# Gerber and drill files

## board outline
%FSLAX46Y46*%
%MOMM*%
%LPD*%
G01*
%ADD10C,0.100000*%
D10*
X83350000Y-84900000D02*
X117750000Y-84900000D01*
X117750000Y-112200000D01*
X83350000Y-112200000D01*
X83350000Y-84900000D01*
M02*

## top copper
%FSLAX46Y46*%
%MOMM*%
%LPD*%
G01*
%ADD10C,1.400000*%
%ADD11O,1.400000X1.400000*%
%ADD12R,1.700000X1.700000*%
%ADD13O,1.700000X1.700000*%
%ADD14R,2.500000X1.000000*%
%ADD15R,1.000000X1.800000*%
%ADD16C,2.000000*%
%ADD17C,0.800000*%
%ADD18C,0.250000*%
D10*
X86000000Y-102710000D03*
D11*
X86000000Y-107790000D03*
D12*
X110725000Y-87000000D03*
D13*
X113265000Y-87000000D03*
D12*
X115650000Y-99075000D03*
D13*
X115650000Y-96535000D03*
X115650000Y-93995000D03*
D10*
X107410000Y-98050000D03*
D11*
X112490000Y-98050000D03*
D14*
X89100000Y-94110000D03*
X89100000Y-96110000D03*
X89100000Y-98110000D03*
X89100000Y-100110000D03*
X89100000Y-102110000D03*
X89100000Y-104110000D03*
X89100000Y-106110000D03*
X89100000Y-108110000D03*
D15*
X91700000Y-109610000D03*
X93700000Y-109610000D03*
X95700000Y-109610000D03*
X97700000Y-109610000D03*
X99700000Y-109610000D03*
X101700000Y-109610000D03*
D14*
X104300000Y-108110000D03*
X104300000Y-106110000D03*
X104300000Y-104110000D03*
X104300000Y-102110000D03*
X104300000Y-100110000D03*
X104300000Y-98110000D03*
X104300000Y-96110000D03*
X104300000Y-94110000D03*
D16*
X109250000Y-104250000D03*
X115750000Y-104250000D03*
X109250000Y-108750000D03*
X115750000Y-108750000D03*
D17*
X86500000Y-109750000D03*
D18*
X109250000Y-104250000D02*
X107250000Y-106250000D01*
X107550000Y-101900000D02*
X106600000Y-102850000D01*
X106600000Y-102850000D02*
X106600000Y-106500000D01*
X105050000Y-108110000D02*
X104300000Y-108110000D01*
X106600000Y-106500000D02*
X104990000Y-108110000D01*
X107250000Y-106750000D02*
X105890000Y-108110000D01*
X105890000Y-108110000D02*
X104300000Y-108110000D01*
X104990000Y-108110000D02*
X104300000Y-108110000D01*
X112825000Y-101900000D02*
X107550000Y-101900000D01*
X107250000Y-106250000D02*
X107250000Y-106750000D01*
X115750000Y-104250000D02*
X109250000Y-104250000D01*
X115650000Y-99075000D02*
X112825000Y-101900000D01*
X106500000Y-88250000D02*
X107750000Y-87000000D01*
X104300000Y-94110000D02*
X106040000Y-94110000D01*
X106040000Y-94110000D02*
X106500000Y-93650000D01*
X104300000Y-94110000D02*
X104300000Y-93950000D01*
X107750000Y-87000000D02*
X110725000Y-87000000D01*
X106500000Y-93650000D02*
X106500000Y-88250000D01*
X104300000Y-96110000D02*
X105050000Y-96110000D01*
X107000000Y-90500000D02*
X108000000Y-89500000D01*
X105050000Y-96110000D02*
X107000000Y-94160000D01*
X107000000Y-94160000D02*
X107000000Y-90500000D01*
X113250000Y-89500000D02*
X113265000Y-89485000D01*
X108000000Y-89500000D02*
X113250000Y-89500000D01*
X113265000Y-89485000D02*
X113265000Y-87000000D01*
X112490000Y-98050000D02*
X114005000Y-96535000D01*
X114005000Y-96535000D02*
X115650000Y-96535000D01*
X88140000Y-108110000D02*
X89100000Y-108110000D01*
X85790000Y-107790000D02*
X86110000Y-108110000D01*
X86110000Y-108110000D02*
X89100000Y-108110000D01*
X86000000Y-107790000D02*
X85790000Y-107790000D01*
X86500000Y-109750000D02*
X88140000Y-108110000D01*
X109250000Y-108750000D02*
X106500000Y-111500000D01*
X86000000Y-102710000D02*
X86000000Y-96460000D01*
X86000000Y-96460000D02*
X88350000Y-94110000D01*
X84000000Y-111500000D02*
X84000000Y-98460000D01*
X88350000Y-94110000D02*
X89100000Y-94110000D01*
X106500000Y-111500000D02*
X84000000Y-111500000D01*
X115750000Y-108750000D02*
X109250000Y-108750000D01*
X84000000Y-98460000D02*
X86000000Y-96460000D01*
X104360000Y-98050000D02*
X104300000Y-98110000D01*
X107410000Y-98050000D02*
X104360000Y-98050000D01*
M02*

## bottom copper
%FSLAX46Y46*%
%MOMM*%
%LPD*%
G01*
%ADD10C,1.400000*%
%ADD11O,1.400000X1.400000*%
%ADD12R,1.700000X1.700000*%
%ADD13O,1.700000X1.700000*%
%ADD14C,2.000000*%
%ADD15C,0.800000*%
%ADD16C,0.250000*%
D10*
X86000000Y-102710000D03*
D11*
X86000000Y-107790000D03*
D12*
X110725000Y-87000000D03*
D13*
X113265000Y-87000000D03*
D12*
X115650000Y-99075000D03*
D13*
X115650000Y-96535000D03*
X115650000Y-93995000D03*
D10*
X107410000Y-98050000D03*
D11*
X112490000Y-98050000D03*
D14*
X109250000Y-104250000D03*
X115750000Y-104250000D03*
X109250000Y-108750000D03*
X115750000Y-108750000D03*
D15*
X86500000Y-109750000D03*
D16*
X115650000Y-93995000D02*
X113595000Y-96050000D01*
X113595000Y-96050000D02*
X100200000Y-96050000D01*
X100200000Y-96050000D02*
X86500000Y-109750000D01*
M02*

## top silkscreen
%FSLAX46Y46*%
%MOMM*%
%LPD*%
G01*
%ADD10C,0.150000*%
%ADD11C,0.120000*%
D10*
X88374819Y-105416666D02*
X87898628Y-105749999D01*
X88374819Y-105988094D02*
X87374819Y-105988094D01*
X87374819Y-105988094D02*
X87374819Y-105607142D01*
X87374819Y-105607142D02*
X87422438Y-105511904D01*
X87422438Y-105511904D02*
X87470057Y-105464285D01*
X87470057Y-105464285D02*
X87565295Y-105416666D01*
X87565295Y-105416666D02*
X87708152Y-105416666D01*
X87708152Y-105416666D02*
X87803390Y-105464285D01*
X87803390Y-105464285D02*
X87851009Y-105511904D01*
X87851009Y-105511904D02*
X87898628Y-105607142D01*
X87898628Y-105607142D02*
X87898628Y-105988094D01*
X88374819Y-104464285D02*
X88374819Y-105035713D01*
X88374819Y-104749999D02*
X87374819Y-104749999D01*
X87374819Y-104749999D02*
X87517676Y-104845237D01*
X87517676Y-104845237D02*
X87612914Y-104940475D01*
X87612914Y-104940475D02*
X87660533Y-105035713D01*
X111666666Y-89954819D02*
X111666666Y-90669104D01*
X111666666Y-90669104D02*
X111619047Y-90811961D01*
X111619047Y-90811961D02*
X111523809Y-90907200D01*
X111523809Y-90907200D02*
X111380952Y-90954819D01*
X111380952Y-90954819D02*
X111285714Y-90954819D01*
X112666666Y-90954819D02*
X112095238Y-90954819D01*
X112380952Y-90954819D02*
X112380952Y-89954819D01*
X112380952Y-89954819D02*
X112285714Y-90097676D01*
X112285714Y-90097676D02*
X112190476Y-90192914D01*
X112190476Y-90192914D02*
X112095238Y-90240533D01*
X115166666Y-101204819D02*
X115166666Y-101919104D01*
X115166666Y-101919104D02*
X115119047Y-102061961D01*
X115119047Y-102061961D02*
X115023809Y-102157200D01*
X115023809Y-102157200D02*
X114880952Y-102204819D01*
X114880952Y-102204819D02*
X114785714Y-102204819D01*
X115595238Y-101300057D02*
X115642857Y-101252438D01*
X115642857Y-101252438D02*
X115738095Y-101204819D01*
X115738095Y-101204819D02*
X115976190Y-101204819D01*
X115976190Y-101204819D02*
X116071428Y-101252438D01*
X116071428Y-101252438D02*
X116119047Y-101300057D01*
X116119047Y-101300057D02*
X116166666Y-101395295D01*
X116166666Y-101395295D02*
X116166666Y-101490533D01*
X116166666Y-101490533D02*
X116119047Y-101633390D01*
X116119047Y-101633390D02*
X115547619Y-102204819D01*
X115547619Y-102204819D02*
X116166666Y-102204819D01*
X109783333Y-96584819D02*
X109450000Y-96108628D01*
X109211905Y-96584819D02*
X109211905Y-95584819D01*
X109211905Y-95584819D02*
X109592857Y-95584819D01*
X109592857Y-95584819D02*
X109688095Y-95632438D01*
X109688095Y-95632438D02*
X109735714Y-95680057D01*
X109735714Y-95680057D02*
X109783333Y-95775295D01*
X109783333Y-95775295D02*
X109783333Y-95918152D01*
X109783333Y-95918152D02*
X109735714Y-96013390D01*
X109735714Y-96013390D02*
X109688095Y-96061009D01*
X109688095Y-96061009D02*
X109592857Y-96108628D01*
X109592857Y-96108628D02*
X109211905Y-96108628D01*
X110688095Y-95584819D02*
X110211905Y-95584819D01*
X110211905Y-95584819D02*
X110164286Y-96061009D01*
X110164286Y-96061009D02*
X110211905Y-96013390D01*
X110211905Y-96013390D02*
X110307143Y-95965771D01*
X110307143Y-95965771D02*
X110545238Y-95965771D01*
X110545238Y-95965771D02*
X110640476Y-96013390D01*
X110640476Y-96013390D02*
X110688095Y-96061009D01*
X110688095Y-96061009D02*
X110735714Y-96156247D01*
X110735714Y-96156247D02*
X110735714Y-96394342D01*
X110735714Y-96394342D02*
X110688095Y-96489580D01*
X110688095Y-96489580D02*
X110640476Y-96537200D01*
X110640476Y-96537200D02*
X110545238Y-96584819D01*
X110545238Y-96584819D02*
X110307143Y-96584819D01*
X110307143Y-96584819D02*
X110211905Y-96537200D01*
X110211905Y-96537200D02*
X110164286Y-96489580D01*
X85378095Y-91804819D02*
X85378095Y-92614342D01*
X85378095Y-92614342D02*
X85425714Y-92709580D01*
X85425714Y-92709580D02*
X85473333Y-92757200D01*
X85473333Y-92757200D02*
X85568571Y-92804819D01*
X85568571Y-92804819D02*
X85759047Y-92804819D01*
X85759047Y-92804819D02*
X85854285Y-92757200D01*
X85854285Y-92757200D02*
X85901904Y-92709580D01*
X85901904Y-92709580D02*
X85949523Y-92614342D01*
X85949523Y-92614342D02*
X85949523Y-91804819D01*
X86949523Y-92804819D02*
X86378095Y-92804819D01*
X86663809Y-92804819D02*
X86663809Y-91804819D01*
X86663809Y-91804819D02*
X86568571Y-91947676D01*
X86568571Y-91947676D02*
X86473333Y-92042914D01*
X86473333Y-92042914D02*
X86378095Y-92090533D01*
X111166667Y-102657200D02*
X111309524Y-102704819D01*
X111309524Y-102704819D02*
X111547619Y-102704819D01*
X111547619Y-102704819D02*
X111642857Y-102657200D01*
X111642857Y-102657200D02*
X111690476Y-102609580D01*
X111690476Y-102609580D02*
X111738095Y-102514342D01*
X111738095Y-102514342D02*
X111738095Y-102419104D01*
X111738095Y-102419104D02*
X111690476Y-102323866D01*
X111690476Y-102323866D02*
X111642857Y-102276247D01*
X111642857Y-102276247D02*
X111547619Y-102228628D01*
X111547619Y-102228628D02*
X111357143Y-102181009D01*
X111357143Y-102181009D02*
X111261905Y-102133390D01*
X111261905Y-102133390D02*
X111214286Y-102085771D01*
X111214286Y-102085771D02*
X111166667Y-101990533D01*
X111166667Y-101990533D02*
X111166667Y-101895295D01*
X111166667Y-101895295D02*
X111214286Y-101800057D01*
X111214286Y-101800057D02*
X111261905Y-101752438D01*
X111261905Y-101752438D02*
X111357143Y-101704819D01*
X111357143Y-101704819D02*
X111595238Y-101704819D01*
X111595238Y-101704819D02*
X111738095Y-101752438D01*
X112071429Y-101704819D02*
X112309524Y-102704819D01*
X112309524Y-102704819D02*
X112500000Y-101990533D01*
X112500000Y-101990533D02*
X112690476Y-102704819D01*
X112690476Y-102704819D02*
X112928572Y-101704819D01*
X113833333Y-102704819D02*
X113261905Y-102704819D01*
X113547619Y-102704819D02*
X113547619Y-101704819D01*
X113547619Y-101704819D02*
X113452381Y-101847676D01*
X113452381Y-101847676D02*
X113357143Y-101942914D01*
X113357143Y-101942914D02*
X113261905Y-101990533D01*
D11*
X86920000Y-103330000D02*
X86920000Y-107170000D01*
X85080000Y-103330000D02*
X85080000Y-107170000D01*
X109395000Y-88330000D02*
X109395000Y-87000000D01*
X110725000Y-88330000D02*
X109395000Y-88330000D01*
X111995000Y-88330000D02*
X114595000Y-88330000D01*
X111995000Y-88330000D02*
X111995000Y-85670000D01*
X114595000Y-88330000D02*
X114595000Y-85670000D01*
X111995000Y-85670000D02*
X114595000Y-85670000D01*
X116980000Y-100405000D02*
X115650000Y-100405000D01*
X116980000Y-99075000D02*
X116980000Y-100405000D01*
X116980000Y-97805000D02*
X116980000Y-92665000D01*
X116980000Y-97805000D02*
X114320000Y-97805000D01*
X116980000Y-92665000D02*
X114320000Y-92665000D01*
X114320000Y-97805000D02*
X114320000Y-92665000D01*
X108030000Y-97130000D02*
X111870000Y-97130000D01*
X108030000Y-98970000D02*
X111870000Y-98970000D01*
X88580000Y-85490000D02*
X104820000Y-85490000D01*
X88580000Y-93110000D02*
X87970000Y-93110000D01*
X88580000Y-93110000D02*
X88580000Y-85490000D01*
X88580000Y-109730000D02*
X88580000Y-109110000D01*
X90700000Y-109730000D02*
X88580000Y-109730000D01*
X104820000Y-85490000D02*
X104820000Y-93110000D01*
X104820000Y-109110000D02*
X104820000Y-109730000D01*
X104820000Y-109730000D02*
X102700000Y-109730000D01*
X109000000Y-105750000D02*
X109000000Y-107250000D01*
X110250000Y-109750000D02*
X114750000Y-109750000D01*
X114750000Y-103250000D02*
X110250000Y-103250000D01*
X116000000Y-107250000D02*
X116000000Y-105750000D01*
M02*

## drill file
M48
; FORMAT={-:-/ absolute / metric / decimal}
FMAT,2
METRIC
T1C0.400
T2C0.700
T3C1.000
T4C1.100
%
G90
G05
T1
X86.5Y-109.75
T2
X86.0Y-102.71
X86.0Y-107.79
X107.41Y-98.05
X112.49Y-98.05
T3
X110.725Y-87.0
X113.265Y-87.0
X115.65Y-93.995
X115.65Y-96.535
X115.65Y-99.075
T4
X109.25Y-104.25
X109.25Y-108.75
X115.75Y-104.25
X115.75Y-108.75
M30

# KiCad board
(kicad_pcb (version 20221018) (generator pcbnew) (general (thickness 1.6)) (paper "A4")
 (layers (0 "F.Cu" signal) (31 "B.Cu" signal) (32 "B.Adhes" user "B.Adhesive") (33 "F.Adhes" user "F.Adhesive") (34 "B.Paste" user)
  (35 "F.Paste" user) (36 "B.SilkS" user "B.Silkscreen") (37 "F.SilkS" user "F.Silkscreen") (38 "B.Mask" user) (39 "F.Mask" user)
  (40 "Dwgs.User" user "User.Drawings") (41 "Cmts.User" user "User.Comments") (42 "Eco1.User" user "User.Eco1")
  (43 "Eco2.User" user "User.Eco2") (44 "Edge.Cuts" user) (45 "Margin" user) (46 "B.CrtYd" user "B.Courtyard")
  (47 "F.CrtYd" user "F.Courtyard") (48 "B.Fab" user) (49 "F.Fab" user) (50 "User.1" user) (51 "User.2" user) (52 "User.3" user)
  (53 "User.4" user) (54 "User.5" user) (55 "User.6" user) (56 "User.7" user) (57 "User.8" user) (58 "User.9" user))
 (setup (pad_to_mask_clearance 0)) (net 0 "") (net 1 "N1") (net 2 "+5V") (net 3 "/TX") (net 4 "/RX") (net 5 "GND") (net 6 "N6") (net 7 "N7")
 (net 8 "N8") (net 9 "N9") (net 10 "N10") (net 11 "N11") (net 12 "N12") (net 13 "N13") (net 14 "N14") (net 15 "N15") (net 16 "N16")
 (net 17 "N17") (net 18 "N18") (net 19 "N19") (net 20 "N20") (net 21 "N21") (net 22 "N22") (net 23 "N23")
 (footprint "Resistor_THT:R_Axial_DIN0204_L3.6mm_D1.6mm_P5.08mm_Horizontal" (layer "F.Cu") (at 86 102.71 -90)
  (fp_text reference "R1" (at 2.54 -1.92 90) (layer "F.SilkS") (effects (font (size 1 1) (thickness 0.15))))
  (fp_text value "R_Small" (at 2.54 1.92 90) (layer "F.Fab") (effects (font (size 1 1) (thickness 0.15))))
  (fp_line (start 0.62 -0.92) (end 4.46 -0.92) (stroke (width 0.12) (type solid)) (layer "F.SilkS"))
  (fp_line (start 0.62 0.92) (end 4.46 0.92) (stroke (width 0.12) (type solid)) (layer "F.SilkS"))
  (pad "1" thru_hole circle (at 0 0 270) (size 1.4 1.4) (drill 0.7) (layers "*.Cu" "*.Mask") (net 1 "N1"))
  (pad "2" thru_hole oval (at 5.08 0 270) (size 1.4 1.4) (drill 0.7) (layers "*.Cu" "*.Mask") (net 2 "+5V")))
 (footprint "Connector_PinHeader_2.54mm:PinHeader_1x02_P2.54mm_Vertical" (layer "F.Cu") (at 110.725 87 90)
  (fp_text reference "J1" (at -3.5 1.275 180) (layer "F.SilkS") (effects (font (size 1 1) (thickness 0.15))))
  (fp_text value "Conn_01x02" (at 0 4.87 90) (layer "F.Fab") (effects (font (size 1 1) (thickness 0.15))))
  (fp_line (start -1.33 -1.33) (end 0 -1.33) (stroke (width 0.12) (type solid)) (layer "F.SilkS"))
  (fp_line (start -1.33 0) (end -1.33 -1.33) (stroke (width 0.12) (type solid)) (layer "F.SilkS"))
  (fp_line (start -1.33 1.27) (end -1.33 3.87) (stroke (width 0.12) (type solid)) (layer "F.SilkS"))
  (fp_line (start -1.33 1.27) (end 1.33 1.27) (stroke (width 0.12) (type solid)) (layer "F.SilkS"))
  (fp_line (start -1.33 3.87) (end 1.33 3.87) (stroke (width 0.12) (type solid)) (layer "F.SilkS"))
  (fp_line (start 1.33 1.27) (end 1.33 3.87) (stroke (width 0.12) (type solid)) (layer "F.SilkS"))
  (pad "1" thru_hole rect (at 0 0 90) (size 1.7 1.7) (drill 1) (layers "*.Cu" "*.Mask") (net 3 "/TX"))
  (pad "2" thru_hole oval (at 0 2.54 90) (size 1.7 1.7) (drill 1) (layers "*.Cu" "*.Mask") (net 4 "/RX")))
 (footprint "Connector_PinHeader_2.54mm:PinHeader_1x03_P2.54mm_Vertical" (layer "F.Cu") (at 115.65 99.075 180)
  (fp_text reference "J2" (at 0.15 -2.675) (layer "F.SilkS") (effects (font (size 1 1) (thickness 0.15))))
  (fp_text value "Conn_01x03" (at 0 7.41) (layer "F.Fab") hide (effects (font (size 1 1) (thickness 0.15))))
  (fp_line (start -1.33 -1.33) (end 0 -1.33) (stroke (width 0.12) (type solid)) (layer "F.SilkS"))
  (fp_line (start -1.33 0) (end -1.33 -1.33) (stroke (width 0.12) (type solid)) (layer "F.SilkS"))
  (fp_line (start -1.33 1.27) (end -1.33 6.41) (stroke (width 0.12) (type solid)) (layer "F.SilkS"))
  (fp_line (start -1.33 1.27) (end 1.33 1.27) (stroke (width 0.12) (type solid)) (layer "F.SilkS"))
  (fp_line (start -1.33 6.41) (end 1.33 6.41) (stroke (width 0.12) (type solid)) (layer "F.SilkS"))
  (fp_line (start 1.33 1.27) (end 1.33 6.41) (stroke (width 0.12) (type solid)) (layer "F.SilkS"))
  (pad "1" thru_hole rect (at 0 0 180) (size 1.7 1.7) (drill 1) (layers "*.Cu" "*.Mask") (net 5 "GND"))
  (pad "2" thru_hole oval (at 0 2.54 180) (size 1.7 1.7) (drill 1) (layers "*.Cu" "*.Mask") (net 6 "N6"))
  (pad "3" thru_hole oval (at 0 5.08 180) (size 1.7 1.7) (drill 1) (layers "*.Cu" "*.Mask") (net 2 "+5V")))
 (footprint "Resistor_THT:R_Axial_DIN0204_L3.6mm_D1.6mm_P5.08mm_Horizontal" (layer "F.Cu") (at 107.41 98.05)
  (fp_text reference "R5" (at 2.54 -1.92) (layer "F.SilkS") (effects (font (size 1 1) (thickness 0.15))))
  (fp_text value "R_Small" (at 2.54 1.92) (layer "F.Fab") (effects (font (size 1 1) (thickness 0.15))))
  (fp_line (start 0.62 -0.92) (end 4.46 -0.92) (stroke (width 0.12) (type solid)) (layer "F.SilkS"))
  (fp_line (start 0.62 0.92) (end 4.46 0.92) (stroke (width 0.12) (type solid)) (layer "F.SilkS"))
  (pad "1" thru_hole circle (at 0 0) (size 1.4 1.4) (drill 0.7) (layers "*.Cu" "*.Mask") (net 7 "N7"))
  (pad "2" thru_hole oval (at 5.08 0) (size 1.4 1.4) (drill 0.7) (layers "*.Cu" "*.Mask") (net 6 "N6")))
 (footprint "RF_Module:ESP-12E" (layer "F.Cu") (at 96.7 97.61)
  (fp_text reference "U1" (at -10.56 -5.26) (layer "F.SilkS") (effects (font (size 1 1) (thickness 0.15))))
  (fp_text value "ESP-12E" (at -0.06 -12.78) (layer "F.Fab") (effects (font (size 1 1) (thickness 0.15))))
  (fp_line (start -8.12 -12.12) (end 8.12 -12.12) (stroke (width 0.12) (type solid)) (layer "F.SilkS"))
  (fp_line (start -8.12 -4.5) (end -8.73 -4.5) (stroke (width 0.12) (type solid)) (layer "F.SilkS"))
  (fp_line (start -8.12 -4.5) (end -8.12 -12.12) (stroke (width 0.12) (type solid)) (layer "F.SilkS"))
  (fp_line (start -8.12 12.12) (end -8.12 11.5) (stroke (width 0.12) (type solid)) (layer "F.SilkS"))
  (fp_line (start -6 12.12) (end -8.12 12.12) (stroke (width 0.12) (type solid)) (layer "F.SilkS"))
  (fp_line (start 8.12 -12.12) (end 8.12 -4.5) (stroke (width 0.12) (type solid)) (layer "F.SilkS"))
  (fp_line (start 8.12 11.5) (end 8.12 12.12) (stroke (width 0.12) (type solid)) (layer "F.SilkS"))
  (fp_line (start 8.12 12.12) (end 6 12.12) (stroke (width 0.12) (type solid)) (layer "F.SilkS"))
  (pad "1" smd rect (at -7.6 -3.5) (size 2.5 1) (layers "F.Cu" "F.Paste" "F.Mask") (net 1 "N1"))
  (pad "2" smd rect (at -7.6 -1.5) (size 2.5 1) (layers "F.Cu" "F.Paste" "F.Mask") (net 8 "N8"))
  (pad "3" smd rect (at -7.6 0.5) (size 2.5 1) (layers "F.Cu" "F.Paste" "F.Mask") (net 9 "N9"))
  (pad "4" smd rect (at -7.6 2.5) (size 2.5 1) (layers "F.Cu" "F.Paste" "F.Mask") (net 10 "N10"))
  (pad "5" smd rect (at -7.6 4.5) (size 2.5 1) (layers "F.Cu" "F.Paste" "F.Mask") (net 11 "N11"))
  (pad "6" smd rect (at -7.6 6.5) (size 2.5 1) (layers "F.Cu" "F.Paste" "F.Mask") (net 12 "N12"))
  (pad "7" smd rect (at -7.6 8.5) (size 2.5 1) (layers "F.Cu" "F.Paste" "F.Mask") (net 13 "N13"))
  (pad "8" smd rect (at -7.6 10.5) (size 2.5 1) (layers "F.Cu" "F.Paste" "F.Mask") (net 2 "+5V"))
  (pad "9" smd rect (at -5 12) (size 1 1.8) (layers "F.Cu" "F.Paste" "F.Mask") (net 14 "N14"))
  (pad "10" smd rect (at -3 12) (size 1 1.8) (layers "F.Cu" "F.Paste" "F.Mask") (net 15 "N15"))
  (pad "11" smd rect (at -1 12) (size 1 1.8) (layers "F.Cu" "F.Paste" "F.Mask") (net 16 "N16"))
  (pad "12" smd rect (at 1 12) (size 1 1.8) (layers "F.Cu" "F.Paste" "F.Mask") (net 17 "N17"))
  (pad "13" smd rect (at 3 12) (size 1 1.8) (layers "F.Cu" "F.Paste" "F.Mask") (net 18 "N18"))
  (pad "14" smd rect (at 5 12) (size 1 1.8) (layers "F.Cu" "F.Paste" "F.Mask") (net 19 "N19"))
  (pad "15" smd rect (at 7.6 10.5) (size 2.5 1) (layers "F.Cu" "F.Paste" "F.Mask") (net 5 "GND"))
  (pad "16" smd rect (at 7.6 8.5) (size 2.5 1) (layers "F.Cu" "F.Paste" "F.Mask") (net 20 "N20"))
  (pad "17" smd rect (at 7.6 6.5) (size 2.5 1) (layers "F.Cu" "F.Paste" "F.Mask") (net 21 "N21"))
  (pad "18" smd rect (at 7.6 4.5) (size 2.5 1) (layers "F.Cu" "F.Paste" "F.Mask") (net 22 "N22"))
  (pad "19" smd rect (at 7.6 2.5) (size 2.5 1) (layers "F.Cu" "F.Paste" "F.Mask") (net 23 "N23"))
  (pad "20" smd rect (at 7.6 0.5) (size 2.5 1) (layers "F.Cu" "F.Paste" "F.Mask") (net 7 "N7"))
  (pad "21" smd rect (at 7.6 -1.5) (size 2.5 1) (layers "F.Cu" "F.Paste" "F.Mask") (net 4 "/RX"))
  (pad "22" smd rect (at 7.6 -3.5) (size 2.5 1) (layers "F.Cu" "F.Paste" "F.Mask") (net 3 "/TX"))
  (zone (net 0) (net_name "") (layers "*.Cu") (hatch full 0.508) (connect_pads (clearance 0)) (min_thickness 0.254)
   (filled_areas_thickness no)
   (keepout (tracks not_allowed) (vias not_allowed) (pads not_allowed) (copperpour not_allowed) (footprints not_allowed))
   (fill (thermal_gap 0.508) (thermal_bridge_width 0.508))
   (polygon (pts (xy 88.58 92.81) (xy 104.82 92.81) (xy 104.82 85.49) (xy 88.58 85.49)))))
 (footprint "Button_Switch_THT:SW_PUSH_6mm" (layer "F.Cu") (at 109.25 104.25)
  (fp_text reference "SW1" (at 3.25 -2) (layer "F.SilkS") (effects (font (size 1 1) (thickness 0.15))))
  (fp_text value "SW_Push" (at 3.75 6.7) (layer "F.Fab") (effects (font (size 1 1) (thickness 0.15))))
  (fp_line (start -0.25 1.5) (end -0.25 3) (stroke (width 0.12) (type solid)) (layer "F.SilkS"))
  (fp_line (start 1 5.5) (end 5.5 5.5) (stroke (width 0.12) (type solid)) (layer "F.SilkS"))
  (fp_line (start 5.5 -1) (end 1 -1) (stroke (width 0.12) (type solid)) (layer "F.SilkS"))
  (fp_line (start 6.75 3) (end 6.75 1.5) (stroke (width 0.12) (type solid)) (layer "F.SilkS"))
  (pad "1" thru_hole circle (at 0 0 90) (size 2 2) (drill 1.1) (layers "*.Cu" "*.Mask") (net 5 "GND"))
  (pad "1" thru_hole circle (at 6.5 0 90) (size 2 2) (drill 1.1) (layers "*.Cu" "*.Mask") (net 5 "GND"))
  (pad "2" thru_hole circle (at 0 4.5 90) (size 2 2) (drill 1.1) (layers "*.Cu" "*.Mask") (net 1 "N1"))
  (pad "2" thru_hole circle (at 6.5 4.5 90) (size 2 2) (drill 1.1) (layers "*.Cu" "*.Mask") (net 1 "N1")))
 (gr_rect (start 83.35 84.9) (end 117.75 112.2) (stroke (width 0.1) (type default)) (fill none) (layer "Edge.Cuts"))
 (segment (start 109.25 104.25) (end 107.25 106.25) (width 0.25) (layer "F.Cu") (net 5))
 (segment (start 107.55 101.9) (end 106.6 102.85) (width 0.25) (layer "F.Cu") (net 5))
 (segment (start 106.6 102.85) (end 106.6 106.5) (width 0.25) (layer "F.Cu") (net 5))
 (segment (start 105.05 108.11) (end 104.3 108.11) (width 0.25) (layer "F.Cu") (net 5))
 (segment (start 106.6 106.5) (end 104.99 108.11) (width 0.25) (layer "F.Cu") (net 5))
 (segment (start 107.25 106.75) (end 105.89 108.11) (width 0.25) (layer "F.Cu") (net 5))
 (segment (start 105.89 108.11) (end 104.3 108.11) (width 0.25) (layer "F.Cu") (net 5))
 (segment (start 104.99 108.11) (end 104.3 108.11) (width 0.25) (layer "F.Cu") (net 5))
 (segment (start 112.825 101.9) (end 107.55 101.9) (width 0.25) (layer "F.Cu") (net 5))
 (segment (start 107.25 106.25) (end 107.25 106.75) (width 0.25) (layer "F.Cu") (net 5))
 (segment (start 115.75 104.25) (end 109.25 104.25) (width 0.25) (layer "F.Cu") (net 5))
 (segment (start 115.65 99.075) (end 112.825 101.9) (width 0.25) (layer "F.Cu") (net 5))
 (segment (start 106.5 88.25) (end 107.75 87) (width 0.25) (layer "F.Cu") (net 3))
 (segment (start 104.3 94.11) (end 106.04 94.11) (width 0.25) (layer "F.Cu") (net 3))
 (segment (start 106.04 94.11) (end 106.5 93.65) (width 0.25) (layer "F.Cu") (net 3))
 (segment (start 104.3 94.11) (end 104.3 93.95) (width 0.25) (layer "F.Cu") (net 3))
 (segment (start 107.75 87) (end 110.725 87) (width 0.25) (layer "F.Cu") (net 3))
 (segment (start 106.5 93.65) (end 106.5 88.25) (width 0.25) (layer "F.Cu") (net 3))
 (segment (start 104.3 96.11) (end 105.05 96.11) (width 0.25) (layer "F.Cu") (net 4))
 (segment (start 107 90.5) (end 108 89.5) (width 0.25) (layer "F.Cu") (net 4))
 (segment (start 105.05 96.11) (end 107 94.16) (width 0.25) (layer "F.Cu") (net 4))
 (segment (start 107 94.16) (end 107 90.5) (width 0.25) (layer "F.Cu") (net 4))
 (segment (start 113.25 89.5) (end 113.265 89.485) (width 0.25) (layer "F.Cu") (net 4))
 (segment (start 108 89.5) (end 113.25 89.5) (width 0.25) (layer "F.Cu") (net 4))
 (segment (start 113.265 89.485) (end 113.265 87) (width 0.25) (layer "F.Cu") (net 4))
 (segment (start 112.49 98.05) (end 114.005 96.535) (width 0.25) (layer "F.Cu") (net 6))
 (segment (start 114.005 96.535) (end 115.65 96.535) (width 0.25) (layer "F.Cu") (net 6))
 (segment (start 88.14 108.11) (end 89.1 108.11) (width 0.25) (layer "F.Cu") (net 2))
 (segment (start 85.79 107.79) (end 86.11 108.11) (width 0.25) (layer "F.Cu") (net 2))
 (segment (start 86.11 108.11) (end 89.1 108.11) (width 0.25) (layer "F.Cu") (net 2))
 (segment (start 86 107.79) (end 85.79 107.79) (width 0.25) (layer "F.Cu") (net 2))
 (segment (start 86.5 109.75) (end 88.14 108.11) (width 0.25) (layer "F.Cu") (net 2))
 (via (at 86.5 109.75) (size 0.8) (drill 0.4) (layers "F.Cu" "B.Cu") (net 2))
 (segment (start 115.65 93.995) (end 113.595 96.05) (width 0.25) (layer "B.Cu") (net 2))
 (segment (start 113.595 96.05) (end 100.2 96.05) (width 0.25) (layer "B.Cu") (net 2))
 (segment (start 100.2 96.05) (end 86.5 109.75) (width 0.25) (layer "B.Cu") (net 2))
 (segment (start 109.25 108.75) (end 106.5 111.5) (width 0.25) (layer "F.Cu") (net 1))
 (segment (start 86 102.71) (end 86 96.46) (width 0.25) (layer "F.Cu") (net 1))
 (segment (start 86 96.46) (end 88.35 94.11) (width 0.25) (layer "F.Cu") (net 1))
 (segment (start 84 111.5) (end 84 98.46) (width 0.25) (layer "F.Cu") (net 1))
 (segment (start 88.35 94.11) (end 89.1 94.11) (width 0.25) (layer "F.Cu") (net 1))
 (segment (start 106.5 111.5) (end 84 111.5) (width 0.25) (layer "F.Cu") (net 1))
 (segment (start 115.75 108.75) (end 109.25 108.75) (width 0.25) (layer "F.Cu") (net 1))
 (segment (start 84 98.46) (end 86 96.46) (width 0.25) (layer "F.Cu") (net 1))
 (segment (start 104.36 98.05) (end 104.3 98.11) (width 0.25) (layer "F.Cu") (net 7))
 (segment (start 107.41 98.05) (end 104.36 98.05) (width 0.25) (layer "F.Cu") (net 7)))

